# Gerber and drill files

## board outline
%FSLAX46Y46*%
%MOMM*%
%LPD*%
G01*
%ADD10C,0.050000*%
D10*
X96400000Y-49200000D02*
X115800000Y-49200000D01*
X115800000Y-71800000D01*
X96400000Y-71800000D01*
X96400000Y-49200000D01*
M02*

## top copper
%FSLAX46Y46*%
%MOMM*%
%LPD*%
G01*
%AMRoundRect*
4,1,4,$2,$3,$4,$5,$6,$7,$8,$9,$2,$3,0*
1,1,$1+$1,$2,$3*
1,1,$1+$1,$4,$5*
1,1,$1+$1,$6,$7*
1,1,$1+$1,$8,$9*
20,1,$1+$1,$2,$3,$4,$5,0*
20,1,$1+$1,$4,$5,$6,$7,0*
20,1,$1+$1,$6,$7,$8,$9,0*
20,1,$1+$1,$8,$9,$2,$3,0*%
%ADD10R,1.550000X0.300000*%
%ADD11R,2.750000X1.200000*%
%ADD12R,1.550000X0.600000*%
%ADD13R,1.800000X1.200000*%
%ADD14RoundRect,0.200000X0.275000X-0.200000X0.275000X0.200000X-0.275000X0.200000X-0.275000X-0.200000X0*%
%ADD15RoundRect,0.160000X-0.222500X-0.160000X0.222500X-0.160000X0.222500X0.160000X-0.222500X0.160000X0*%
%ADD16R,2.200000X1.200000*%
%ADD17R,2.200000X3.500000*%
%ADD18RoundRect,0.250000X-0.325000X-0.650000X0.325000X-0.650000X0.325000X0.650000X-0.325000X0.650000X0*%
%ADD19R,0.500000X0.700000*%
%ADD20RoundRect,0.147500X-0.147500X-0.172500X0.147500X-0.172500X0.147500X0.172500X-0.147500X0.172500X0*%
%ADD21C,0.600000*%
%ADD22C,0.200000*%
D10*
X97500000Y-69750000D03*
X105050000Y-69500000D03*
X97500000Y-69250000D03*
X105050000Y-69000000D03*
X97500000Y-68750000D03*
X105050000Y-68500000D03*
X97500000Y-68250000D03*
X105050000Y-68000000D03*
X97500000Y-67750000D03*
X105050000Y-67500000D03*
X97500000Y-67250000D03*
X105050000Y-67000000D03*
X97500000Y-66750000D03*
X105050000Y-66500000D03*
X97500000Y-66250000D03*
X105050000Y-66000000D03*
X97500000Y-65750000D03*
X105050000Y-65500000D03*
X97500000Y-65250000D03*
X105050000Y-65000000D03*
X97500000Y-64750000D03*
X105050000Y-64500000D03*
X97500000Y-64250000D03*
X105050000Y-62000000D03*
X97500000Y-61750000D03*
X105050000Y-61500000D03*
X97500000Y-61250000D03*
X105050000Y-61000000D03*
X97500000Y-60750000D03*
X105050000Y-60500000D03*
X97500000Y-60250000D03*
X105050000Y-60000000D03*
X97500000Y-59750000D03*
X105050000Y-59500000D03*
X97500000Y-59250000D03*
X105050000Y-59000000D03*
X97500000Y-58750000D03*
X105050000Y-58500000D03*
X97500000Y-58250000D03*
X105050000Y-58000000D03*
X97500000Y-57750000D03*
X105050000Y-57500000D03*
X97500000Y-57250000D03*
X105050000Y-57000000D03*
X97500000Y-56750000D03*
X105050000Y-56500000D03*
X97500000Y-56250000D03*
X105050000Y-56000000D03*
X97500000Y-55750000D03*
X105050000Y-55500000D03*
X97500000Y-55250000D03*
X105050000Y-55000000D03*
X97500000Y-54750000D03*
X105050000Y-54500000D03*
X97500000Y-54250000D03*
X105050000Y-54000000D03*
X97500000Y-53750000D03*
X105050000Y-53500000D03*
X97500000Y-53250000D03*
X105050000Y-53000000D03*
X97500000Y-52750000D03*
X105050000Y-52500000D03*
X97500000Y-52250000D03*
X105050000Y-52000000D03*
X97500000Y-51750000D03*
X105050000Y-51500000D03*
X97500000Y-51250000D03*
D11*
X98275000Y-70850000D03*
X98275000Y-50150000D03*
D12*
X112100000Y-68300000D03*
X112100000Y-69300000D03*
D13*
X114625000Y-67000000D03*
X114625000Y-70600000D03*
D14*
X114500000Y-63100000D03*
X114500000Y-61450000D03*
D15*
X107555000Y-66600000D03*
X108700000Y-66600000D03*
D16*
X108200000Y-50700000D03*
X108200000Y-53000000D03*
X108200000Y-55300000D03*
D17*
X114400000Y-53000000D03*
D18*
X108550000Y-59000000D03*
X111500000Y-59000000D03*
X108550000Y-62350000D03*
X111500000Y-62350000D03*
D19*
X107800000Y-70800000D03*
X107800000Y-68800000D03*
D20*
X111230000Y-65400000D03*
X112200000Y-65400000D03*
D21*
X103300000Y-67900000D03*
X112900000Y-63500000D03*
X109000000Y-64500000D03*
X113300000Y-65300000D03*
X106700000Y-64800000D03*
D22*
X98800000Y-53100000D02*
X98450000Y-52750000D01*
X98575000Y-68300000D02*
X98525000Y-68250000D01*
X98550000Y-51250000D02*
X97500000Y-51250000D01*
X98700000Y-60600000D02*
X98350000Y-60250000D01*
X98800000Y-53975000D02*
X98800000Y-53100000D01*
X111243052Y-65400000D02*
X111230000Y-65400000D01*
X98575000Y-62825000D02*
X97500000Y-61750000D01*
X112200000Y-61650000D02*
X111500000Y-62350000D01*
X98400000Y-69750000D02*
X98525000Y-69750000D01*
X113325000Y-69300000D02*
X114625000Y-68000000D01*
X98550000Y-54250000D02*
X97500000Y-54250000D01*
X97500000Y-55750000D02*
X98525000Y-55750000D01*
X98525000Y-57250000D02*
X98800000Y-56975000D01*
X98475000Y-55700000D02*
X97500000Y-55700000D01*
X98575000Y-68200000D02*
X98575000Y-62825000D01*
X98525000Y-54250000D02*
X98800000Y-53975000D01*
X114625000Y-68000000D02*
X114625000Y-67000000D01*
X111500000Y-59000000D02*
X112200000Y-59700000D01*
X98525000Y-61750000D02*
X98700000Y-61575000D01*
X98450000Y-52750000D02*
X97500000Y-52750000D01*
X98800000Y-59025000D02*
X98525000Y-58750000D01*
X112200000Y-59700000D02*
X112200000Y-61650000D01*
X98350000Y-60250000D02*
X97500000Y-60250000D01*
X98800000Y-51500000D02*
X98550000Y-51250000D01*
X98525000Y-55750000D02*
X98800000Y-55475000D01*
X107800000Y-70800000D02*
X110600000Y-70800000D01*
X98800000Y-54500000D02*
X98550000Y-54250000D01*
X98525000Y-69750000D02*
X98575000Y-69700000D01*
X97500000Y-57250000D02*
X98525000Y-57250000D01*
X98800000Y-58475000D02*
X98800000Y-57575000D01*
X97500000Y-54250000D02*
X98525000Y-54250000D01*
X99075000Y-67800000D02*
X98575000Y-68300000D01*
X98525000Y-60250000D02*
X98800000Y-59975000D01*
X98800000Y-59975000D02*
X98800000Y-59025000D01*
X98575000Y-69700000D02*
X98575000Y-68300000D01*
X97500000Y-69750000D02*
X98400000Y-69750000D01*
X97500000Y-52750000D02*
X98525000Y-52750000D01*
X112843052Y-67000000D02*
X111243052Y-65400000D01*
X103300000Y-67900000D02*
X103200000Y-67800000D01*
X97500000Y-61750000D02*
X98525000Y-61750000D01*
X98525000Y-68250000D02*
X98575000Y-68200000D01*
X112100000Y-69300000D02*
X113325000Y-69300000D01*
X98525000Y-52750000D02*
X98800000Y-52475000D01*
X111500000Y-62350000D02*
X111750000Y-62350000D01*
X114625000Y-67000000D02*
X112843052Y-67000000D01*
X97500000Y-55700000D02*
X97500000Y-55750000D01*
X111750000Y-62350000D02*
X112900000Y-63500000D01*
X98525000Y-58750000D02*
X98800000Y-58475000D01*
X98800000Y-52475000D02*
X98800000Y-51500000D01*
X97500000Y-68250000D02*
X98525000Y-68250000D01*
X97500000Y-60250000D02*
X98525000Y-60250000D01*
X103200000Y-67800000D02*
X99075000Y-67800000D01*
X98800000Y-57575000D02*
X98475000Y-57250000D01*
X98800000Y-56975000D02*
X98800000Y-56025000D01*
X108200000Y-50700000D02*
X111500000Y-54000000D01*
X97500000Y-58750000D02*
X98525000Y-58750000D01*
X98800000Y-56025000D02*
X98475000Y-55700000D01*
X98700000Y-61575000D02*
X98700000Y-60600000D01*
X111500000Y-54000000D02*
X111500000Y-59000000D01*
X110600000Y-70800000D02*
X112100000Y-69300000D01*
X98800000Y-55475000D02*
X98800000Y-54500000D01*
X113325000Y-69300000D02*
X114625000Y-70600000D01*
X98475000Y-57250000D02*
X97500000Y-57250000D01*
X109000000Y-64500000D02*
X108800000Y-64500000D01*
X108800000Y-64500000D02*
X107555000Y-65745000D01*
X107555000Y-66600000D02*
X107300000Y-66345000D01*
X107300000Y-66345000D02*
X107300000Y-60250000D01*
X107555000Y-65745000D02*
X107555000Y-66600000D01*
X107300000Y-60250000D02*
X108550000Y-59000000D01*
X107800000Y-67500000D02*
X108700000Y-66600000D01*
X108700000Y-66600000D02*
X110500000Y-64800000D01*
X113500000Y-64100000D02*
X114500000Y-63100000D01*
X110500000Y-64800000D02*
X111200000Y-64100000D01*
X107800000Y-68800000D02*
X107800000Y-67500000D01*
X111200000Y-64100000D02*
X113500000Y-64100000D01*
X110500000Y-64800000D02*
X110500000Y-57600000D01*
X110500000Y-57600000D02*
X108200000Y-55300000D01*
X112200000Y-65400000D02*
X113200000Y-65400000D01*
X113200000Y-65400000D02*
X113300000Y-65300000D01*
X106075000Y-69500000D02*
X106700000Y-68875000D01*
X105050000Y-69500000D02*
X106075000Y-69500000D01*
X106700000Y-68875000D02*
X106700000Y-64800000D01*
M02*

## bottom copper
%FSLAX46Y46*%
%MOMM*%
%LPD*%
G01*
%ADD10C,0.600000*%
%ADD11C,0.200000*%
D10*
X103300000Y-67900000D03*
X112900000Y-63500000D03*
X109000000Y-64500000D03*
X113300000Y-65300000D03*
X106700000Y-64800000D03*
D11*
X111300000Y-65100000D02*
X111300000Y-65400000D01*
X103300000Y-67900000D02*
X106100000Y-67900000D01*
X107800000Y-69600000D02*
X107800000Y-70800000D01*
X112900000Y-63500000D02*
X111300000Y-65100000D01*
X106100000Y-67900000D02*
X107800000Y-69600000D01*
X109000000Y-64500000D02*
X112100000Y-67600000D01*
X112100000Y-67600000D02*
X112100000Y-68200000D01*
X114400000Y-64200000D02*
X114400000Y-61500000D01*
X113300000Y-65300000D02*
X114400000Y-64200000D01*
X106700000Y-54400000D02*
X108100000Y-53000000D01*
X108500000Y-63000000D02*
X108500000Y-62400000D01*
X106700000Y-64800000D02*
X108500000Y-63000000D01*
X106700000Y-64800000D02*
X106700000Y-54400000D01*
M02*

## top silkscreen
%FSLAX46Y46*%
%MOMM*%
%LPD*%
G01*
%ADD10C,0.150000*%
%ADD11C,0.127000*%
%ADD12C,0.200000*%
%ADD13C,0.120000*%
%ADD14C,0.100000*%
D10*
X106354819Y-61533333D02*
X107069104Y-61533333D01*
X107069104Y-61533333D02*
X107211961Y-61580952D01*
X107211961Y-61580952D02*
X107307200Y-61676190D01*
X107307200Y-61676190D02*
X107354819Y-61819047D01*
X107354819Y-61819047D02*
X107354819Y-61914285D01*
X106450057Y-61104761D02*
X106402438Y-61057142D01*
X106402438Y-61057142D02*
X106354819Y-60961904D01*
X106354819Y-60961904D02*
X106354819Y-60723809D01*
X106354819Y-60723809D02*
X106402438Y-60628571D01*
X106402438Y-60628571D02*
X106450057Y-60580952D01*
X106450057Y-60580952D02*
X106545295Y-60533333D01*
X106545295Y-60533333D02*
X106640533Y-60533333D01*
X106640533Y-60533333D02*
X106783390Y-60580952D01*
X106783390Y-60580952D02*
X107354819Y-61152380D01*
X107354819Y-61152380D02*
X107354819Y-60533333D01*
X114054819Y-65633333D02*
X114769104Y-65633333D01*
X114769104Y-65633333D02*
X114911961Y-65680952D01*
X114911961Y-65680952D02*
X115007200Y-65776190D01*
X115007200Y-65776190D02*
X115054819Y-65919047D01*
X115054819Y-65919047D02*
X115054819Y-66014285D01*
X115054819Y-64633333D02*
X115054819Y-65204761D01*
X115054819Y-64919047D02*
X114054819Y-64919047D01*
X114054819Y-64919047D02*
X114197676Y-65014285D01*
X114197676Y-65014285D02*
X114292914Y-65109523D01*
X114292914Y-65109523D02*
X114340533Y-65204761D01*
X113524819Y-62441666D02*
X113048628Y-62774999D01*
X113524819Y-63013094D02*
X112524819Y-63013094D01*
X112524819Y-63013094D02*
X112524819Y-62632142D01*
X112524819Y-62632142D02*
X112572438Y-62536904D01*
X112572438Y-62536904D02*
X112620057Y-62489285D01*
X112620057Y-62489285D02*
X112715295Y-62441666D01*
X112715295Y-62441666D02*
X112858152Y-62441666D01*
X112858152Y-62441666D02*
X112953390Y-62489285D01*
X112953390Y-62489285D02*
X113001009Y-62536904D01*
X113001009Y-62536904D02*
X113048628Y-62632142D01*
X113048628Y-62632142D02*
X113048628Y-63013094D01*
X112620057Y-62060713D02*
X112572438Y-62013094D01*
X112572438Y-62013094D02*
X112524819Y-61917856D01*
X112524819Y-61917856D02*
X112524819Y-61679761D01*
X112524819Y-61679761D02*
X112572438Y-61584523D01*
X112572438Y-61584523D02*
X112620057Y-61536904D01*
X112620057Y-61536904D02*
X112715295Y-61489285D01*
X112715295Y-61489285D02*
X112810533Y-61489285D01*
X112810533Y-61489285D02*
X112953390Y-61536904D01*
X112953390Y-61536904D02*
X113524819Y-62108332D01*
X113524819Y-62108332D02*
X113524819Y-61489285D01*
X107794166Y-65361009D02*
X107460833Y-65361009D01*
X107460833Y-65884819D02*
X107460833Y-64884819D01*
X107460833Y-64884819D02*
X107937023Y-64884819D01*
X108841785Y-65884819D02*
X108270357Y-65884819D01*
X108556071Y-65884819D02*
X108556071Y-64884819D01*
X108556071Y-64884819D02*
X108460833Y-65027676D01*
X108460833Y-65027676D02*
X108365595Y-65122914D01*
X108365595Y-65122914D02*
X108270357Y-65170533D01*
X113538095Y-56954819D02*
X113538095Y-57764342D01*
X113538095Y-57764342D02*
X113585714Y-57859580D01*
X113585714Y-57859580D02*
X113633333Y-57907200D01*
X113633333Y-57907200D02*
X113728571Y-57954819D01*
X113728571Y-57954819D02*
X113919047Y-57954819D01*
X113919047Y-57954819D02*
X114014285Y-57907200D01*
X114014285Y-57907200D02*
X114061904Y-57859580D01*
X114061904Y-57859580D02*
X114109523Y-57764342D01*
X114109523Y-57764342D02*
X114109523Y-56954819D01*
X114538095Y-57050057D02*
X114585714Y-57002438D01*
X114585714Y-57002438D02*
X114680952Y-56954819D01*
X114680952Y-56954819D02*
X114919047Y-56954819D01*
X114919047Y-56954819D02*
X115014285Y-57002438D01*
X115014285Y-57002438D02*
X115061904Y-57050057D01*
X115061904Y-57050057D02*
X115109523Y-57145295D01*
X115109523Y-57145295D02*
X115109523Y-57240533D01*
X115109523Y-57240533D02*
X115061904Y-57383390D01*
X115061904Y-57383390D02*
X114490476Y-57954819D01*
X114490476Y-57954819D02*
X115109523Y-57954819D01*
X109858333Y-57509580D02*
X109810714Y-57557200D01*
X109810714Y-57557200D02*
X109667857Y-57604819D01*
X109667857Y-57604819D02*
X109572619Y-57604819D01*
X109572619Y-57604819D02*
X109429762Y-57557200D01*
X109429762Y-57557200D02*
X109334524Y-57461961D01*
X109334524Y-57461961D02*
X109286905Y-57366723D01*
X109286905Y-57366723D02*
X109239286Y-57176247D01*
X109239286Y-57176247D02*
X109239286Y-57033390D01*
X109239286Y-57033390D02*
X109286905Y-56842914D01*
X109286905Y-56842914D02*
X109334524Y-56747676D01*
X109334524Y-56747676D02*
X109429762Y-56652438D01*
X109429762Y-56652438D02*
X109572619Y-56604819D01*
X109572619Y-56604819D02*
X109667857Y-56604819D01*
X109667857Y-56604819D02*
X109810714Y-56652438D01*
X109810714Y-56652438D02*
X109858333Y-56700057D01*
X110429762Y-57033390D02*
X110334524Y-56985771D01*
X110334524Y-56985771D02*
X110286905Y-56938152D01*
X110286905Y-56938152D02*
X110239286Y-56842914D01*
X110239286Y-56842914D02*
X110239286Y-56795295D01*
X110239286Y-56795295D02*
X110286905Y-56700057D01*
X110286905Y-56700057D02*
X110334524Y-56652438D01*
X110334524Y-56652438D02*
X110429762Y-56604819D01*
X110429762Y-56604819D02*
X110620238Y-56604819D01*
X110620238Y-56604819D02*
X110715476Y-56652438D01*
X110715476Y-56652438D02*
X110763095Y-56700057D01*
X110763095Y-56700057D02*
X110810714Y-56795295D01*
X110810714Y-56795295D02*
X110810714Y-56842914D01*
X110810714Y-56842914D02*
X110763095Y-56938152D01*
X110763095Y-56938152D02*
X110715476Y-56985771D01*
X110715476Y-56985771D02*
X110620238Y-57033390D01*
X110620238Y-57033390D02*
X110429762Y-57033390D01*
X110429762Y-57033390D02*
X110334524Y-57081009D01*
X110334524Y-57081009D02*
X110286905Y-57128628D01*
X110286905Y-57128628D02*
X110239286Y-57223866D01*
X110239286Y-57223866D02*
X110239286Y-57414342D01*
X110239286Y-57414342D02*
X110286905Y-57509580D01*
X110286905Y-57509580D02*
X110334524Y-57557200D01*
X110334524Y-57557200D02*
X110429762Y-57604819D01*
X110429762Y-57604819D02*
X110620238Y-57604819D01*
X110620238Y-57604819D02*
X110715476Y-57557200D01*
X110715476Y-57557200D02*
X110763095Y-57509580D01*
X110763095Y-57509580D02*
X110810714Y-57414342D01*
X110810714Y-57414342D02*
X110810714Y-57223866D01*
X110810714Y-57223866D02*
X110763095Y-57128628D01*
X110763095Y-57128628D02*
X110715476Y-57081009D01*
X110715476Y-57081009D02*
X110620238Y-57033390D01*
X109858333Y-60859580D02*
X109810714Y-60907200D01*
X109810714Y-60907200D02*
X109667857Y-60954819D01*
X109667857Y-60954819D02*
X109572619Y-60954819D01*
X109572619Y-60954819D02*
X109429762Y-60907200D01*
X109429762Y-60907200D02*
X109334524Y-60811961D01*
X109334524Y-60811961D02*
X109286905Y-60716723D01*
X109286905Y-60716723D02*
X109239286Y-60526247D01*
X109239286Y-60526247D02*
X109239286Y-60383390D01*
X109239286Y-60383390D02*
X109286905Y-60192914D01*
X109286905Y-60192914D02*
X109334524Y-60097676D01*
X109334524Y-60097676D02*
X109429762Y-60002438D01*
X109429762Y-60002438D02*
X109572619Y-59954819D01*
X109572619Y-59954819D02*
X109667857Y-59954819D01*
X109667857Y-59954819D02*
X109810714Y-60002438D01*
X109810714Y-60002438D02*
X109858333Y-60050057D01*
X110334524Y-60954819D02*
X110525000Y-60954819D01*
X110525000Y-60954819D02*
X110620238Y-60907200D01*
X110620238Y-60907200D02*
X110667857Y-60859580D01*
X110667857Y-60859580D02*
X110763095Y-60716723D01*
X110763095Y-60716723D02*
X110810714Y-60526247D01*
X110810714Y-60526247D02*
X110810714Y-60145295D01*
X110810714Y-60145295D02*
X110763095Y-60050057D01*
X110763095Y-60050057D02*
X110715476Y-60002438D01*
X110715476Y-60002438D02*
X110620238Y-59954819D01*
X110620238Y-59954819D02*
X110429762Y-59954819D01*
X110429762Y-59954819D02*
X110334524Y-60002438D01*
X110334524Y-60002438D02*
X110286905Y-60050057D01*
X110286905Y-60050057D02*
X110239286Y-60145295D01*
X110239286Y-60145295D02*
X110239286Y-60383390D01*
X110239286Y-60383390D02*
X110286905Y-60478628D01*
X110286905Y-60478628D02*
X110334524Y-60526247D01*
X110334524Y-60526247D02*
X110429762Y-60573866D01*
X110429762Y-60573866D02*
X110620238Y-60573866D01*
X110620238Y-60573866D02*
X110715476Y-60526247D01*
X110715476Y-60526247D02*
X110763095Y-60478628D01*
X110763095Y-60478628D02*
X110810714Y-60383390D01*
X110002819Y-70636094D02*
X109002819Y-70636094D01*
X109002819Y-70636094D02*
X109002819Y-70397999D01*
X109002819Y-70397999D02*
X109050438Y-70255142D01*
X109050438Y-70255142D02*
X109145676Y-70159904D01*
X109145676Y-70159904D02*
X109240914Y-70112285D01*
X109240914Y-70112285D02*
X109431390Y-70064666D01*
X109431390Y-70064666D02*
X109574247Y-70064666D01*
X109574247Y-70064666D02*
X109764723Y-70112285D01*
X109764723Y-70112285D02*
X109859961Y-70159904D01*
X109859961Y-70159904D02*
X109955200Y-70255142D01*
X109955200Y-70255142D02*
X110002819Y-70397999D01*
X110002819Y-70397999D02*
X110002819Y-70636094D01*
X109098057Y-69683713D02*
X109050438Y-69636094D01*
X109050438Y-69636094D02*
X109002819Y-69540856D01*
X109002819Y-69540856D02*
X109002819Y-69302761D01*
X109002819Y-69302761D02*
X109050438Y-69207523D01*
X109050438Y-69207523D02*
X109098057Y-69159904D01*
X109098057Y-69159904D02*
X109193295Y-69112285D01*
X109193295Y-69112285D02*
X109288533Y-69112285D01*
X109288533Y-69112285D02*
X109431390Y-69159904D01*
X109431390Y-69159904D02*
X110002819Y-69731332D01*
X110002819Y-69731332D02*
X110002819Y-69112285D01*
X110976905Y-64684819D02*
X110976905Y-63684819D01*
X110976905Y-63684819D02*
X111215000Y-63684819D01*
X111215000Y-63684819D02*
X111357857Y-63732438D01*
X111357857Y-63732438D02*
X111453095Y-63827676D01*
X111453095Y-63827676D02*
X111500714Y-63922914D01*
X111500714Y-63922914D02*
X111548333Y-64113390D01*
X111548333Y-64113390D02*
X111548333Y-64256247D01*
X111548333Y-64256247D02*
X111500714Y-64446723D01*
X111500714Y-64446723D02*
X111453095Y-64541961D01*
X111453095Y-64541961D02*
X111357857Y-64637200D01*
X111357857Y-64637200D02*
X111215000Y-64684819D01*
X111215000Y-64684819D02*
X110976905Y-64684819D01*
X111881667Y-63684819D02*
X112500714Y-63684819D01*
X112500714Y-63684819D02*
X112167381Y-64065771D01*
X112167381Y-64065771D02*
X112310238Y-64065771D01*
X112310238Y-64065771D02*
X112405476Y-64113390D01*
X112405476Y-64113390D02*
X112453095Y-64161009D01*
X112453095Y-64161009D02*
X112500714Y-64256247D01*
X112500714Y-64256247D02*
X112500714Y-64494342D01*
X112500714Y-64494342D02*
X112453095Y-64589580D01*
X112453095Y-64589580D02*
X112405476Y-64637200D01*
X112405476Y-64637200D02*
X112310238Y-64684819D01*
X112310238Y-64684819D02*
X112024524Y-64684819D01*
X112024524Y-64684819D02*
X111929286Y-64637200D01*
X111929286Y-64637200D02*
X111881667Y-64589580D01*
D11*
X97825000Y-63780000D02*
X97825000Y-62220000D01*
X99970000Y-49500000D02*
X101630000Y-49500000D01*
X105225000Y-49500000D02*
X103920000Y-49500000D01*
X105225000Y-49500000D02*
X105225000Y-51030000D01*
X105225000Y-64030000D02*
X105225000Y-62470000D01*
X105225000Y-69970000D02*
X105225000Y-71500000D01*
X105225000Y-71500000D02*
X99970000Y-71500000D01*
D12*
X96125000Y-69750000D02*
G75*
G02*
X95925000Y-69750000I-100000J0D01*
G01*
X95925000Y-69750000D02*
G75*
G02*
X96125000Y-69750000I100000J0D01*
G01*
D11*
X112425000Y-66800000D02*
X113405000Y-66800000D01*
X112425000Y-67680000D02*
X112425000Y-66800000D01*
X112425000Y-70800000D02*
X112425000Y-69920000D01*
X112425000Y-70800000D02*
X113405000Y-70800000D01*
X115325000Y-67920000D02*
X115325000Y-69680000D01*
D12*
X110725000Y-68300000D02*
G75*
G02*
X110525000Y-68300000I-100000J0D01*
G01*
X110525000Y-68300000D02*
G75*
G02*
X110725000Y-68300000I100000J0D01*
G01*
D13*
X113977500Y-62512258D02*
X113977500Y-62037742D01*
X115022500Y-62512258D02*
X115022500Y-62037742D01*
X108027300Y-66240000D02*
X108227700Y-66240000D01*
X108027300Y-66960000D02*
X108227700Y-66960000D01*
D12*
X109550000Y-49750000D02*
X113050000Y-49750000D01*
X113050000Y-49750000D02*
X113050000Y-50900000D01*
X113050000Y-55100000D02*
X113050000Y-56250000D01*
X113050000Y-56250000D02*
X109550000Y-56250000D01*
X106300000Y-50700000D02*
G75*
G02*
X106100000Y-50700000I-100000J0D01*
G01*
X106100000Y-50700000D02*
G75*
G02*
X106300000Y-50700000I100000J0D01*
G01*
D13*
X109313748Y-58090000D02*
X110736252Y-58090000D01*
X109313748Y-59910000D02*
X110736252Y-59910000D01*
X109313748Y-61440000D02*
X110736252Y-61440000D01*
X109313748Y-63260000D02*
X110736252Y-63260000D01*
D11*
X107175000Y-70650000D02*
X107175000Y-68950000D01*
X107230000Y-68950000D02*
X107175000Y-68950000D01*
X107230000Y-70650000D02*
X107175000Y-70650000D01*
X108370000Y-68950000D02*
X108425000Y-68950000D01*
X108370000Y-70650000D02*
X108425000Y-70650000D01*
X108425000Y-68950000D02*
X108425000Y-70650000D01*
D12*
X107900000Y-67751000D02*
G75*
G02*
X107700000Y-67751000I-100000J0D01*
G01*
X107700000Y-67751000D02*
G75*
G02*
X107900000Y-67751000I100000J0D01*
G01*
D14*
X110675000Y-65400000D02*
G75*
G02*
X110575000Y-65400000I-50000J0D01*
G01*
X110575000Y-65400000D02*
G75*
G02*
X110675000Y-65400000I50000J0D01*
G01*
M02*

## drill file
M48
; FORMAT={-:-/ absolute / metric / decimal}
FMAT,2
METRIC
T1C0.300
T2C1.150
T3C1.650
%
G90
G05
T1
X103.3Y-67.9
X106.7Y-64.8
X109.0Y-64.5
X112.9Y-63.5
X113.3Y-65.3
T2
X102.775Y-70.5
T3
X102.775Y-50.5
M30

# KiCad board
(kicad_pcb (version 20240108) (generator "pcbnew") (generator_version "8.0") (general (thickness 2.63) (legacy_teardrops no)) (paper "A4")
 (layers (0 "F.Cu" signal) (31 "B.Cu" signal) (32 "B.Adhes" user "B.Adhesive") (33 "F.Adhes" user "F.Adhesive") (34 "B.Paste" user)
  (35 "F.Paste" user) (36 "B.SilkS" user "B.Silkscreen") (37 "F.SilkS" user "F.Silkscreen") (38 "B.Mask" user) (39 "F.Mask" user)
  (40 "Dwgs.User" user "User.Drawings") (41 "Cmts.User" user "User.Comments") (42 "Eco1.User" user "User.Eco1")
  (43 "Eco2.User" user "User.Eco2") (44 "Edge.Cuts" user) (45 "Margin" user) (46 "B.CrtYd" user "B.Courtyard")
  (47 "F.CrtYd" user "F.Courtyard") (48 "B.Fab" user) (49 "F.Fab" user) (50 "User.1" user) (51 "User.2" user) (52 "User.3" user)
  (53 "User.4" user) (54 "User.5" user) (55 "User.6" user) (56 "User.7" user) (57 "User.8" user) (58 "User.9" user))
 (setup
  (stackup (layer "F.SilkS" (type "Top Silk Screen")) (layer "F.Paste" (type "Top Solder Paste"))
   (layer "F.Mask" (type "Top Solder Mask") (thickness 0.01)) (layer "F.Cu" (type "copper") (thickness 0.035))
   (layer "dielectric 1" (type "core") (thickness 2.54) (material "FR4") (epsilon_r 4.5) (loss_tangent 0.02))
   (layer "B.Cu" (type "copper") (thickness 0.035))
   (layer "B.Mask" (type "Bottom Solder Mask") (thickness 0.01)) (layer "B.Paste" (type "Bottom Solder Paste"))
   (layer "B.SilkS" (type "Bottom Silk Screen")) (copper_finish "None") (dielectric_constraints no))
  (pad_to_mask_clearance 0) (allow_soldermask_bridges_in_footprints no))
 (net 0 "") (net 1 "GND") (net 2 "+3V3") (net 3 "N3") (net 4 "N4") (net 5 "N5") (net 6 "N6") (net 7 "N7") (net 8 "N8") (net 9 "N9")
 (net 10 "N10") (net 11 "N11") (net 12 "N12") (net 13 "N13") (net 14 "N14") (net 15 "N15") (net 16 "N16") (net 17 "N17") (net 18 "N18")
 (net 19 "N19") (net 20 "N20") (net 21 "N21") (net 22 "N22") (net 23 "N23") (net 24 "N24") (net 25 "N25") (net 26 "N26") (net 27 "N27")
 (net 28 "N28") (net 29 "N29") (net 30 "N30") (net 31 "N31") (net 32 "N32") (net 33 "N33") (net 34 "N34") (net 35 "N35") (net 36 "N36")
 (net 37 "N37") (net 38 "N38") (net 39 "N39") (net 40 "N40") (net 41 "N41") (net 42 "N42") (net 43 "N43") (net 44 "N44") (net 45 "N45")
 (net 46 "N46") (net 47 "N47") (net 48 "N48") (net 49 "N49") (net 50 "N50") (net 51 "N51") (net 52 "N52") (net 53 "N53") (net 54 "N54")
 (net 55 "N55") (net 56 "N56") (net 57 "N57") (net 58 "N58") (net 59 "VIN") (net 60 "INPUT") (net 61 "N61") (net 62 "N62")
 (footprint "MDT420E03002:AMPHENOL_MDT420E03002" (layer "F.Cu") (at 102.775 60.5 90)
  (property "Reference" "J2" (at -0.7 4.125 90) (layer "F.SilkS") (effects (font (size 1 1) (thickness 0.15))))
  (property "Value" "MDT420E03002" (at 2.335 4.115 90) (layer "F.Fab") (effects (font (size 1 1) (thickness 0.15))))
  (fp_line (start -3.28 -4.95) (end -1.72 -4.95) (stroke (width 0.127) (type solid)) (layer "F.SilkS"))
  (fp_line (start 11 -2.805) (end 11 -1.145) (stroke (width 0.127) (type solid)) (layer "F.SilkS"))
  (fp_line (start 11 2.45) (end 11 1.145) (stroke (width 0.127) (type solid)) (layer "F.SilkS"))
  (fp_line (start 11 2.45) (end 9.47 2.45) (stroke (width 0.127) (type solid)) (layer "F.SilkS"))
  (fp_line (start -3.53 2.45) (end -1.97 2.45) (stroke (width 0.127) (type solid)) (layer "F.SilkS"))
  (fp_line (start -9.47 2.45) (end -11 2.45) (stroke (width 0.127) (type solid)) (layer "F.SilkS"))
  (fp_line (start -11 2.45) (end -11 -2.805) (stroke (width 0.127) (type solid)) (layer "F.SilkS"))
  (fp_circle (center -9.25 -6.75) (end -9.15 -6.75) (stroke (width 0.2) (type solid)) (fill none) (layer "F.SilkS"))
  (pad "" np_thru_hole circle (at -10 0 90) (size 1.15 1.15) (drill 1.15) (layers "*.Cu" "*.Mask"))
  (pad "" np_thru_hole circle (at 10 0 90) (size 1.65 1.65) (drill 1.65) (layers "*.Cu" "*.Mask"))
  (pad "1" smd rect (at -9.25 -5.275 90) (size 0.3 1.55) (layers "F.Cu" "F.Paste" "F.Mask") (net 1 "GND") (solder_mask_margin 0.102))
  (pad "2" smd rect (at -9 2.275 90) (size 0.3 1.55) (layers "F.Cu" "F.Paste" "F.Mask") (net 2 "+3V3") (solder_mask_margin 0.102))
  (pad "3" smd rect (at -8.75 -5.275 90) (size 0.3 1.55) (layers "F.Cu" "F.Paste" "F.Mask") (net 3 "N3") (solder_mask_margin 0.102))
  (pad "4" smd rect (at -8.5 2.275 90) (size 0.3 1.55) (layers "F.Cu" "F.Paste" "F.Mask") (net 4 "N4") (solder_mask_margin 0.102))
  (pad "5" smd rect (at -8.25 -5.275 90) (size 0.3 1.55) (layers "F.Cu" "F.Paste" "F.Mask") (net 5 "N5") (solder_mask_margin 0.102))
  (pad "6" smd rect (at -8 2.275 90) (size 0.3 1.55) (layers "F.Cu" "F.Paste" "F.Mask") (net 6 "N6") (solder_mask_margin 0.102))
  (pad "7" smd rect (at -7.75 -5.275 90) (size 0.3 1.55) (layers "F.Cu" "F.Paste" "F.Mask") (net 1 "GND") (solder_mask_margin 0.102))
  (pad "8" smd rect (at -7.5 2.275 90) (size 0.3 1.55) (layers "F.Cu" "F.Paste" "F.Mask") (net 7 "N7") (solder_mask_margin 0.102))
  (pad "9" smd rect (at -7.25 -5.275 90) (size 0.3 1.55) (layers "F.Cu" "F.Paste" "F.Mask") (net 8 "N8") (solder_mask_margin 0.102))
  (pad "10" smd rect (at -7 2.275 90) (size 0.3 1.55) (layers "F.Cu" "F.Paste" "F.Mask") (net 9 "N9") (solder_mask_margin 0.102))
  (pad "11" smd rect (at -6.75 -5.275 90) (size 0.3 1.55) (layers "F.Cu" "F.Paste" "F.Mask") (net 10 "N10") (solder_mask_margin 0.102))
  (pad "12" smd rect (at -6.5 2.275 90) (size 0.3 1.55) (layers "F.Cu" "F.Paste" "F.Mask") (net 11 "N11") (solder_mask_margin 0.102))
  (pad "13" smd rect (at -6.25 -5.275 90) (size 0.3 1.55) (layers "F.Cu" "F.Paste" "F.Mask") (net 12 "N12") (solder_mask_margin 0.102))
  (pad "14" smd rect (at -6 2.275 90) (size 0.3 1.55) (layers "F.Cu" "F.Paste" "F.Mask") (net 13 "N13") (solder_mask_margin 0.102))
  (pad "15" smd rect (at -5.75 -5.275 90) (size 0.3 1.55) (layers "F.Cu" "F.Paste" "F.Mask") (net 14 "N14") (solder_mask_margin 0.102))
  (pad "16" smd rect (at -5.5 2.275 90) (size 0.3 1.55) (layers "F.Cu" "F.Paste" "F.Mask") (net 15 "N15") (solder_mask_margin 0.102))
  (pad "17" smd rect (at -5.25 -5.275 90) (size 0.3 1.55) (layers "F.Cu" "F.Paste" "F.Mask") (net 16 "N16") (solder_mask_margin 0.102))
  (pad "18" smd rect (at -5 2.275 90) (size 0.3 1.55) (layers "F.Cu" "F.Paste" "F.Mask") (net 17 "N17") (solder_mask_margin 0.102))
  (pad "19" smd rect (at -4.75 -5.275 90) (size 0.3 1.55) (layers "F.Cu" "F.Paste" "F.Mask") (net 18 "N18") (solder_mask_margin 0.102))
  (pad "20" smd rect (at -4.5 2.275 90) (size 0.3 1.55) (layers "F.Cu" "F.Paste" "F.Mask") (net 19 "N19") (solder_mask_margin 0.102))
  (pad "21" smd rect (at -4.25 -5.275 90) (size 0.3 1.55) (layers "F.Cu" "F.Paste" "F.Mask") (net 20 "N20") (solder_mask_margin 0.102))
  (pad "22" smd rect (at -4 2.275 90) (size 0.3 1.55) (layers "F.Cu" "F.Paste" "F.Mask") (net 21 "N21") (solder_mask_margin 0.102))
  (pad "23" smd rect (at -3.75 -5.275 90) (size 0.3 1.55) (layers "F.Cu" "F.Paste" "F.Mask") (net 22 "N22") (solder_mask_margin 0.102))
  (pad "32" smd rect (at -1.5 2.275 90) (size 0.3 1.55) (layers "F.Cu" "F.Paste" "F.Mask") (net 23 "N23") (solder_mask_margin 0.102))
  (pad "33" smd rect (at -1.25 -5.275 90) (size 0.3 1.55) (layers "F.Cu" "F.Paste" "F.Mask") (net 1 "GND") (solder_mask_margin 0.102))
  (pad "34" smd rect (at -1 2.275 90) (size 0.3 1.55) (layers "F.Cu" "F.Paste" "F.Mask") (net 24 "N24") (solder_mask_margin 0.102))
  (pad "35" smd rect (at -0.75 -5.275 90) (size 0.3 1.55) (layers "F.Cu" "F.Paste" "F.Mask") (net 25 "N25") (solder_mask_margin 0.102))
  (pad "36" smd rect (at -0.5 2.275 90) (size 0.3 1.55) (layers "F.Cu" "F.Paste" "F.Mask") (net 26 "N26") (solder_mask_margin 0.102))
  (pad "37" smd rect (at -0.25 -5.275 90) (size 0.3 1.55) (layers "F.Cu" "F.Paste" "F.Mask") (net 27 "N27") (solder_mask_margin 0.102))
  (pad "38" smd rect (at 0 2.275 90) (size 0.3 1.55) (layers "F.Cu" "F.Paste" "F.Mask") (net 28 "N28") (solder_mask_margin 0.102))
  (pad "39" smd rect (at 0.25 -5.275 90) (size 0.3 1.55) (layers "F.Cu" "F.Paste" "F.Mask") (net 1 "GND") (solder_mask_margin 0.102))
  (pad "40" smd rect (at 0.5 2.275 90) (size 0.3 1.55) (layers "F.Cu" "F.Paste" "F.Mask") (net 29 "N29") (solder_mask_margin 0.102))
  (pad "41" smd rect (at 0.75 -5.275 90) (size 0.3 1.55) (layers "F.Cu" "F.Paste" "F.Mask") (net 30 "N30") (solder_mask_margin 0.102))
  (pad "42" smd rect (at 1 2.275 90) (size 0.3 1.55) (layers "F.Cu" "F.Paste" "F.Mask") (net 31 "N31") (solder_mask_margin 0.102))
  (pad "43" smd rect (at 1.25 -5.275 90) (size 0.3 1.55) (layers "F.Cu" "F.Paste" "F.Mask") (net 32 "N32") (solder_mask_margin 0.102))
  (pad "44" smd rect (at 1.5 2.275 90) (size 0.3 1.55) (layers "F.Cu" "F.Paste" "F.Mask") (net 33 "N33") (solder_mask_margin 0.102))
  (pad "45" smd rect (at 1.75 -5.275 90) (size 0.3 1.55) (layers "F.Cu" "F.Paste" "F.Mask") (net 1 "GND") (solder_mask_margin 0.102))
  (pad "46" smd rect (at 2 2.275 90) (size 0.3 1.55) (layers "F.Cu" "F.Paste" "F.Mask") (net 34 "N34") (solder_mask_margin 0.102))
  (pad "47" smd rect (at 2.25 -5.275 90) (size 0.3 1.55) (layers "F.Cu" "F.Paste" "F.Mask") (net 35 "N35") (solder_mask_margin 0.102))
  (pad "48" smd rect (at 2.5 2.275 90) (size 0.3 1.55) (layers "F.Cu" "F.Paste" "F.Mask") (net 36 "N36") (solder_mask_margin 0.102))
  (pad "49" smd rect (at 2.75 -5.275 90) (size 0.3 1.55) (layers "F.Cu" "F.Paste" "F.Mask") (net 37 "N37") (solder_mask_margin 0.102))
  (pad "50" smd rect (at 3 2.275 90) (size 0.3 1.55) (layers "F.Cu" "F.Paste" "F.Mask") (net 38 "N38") (solder_mask_margin 0.102))
  (pad "51" smd rect (at 3.25 -5.275 90) (size 0.3 1.55) (layers "F.Cu" "F.Paste" "F.Mask") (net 1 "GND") (solder_mask_margin 0.102))
  (pad "52" smd rect (at 3.5 2.275 90) (size 0.3 1.55) (layers "F.Cu" "F.Paste" "F.Mask") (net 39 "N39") (solder_mask_margin 0.102))
  (pad "53" smd rect (at 3.75 -5.275 90) (size 0.3 1.55) (layers "F.Cu" "F.Paste" "F.Mask") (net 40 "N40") (solder_mask_margin 0.102))
  (pad "54" smd rect (at 4 2.275 90) (size 0.3 1.55) (layers "F.Cu" "F.Paste" "F.Mask") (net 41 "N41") (solder_mask_margin 0.102))
  (pad "55" smd rect (at 4.25 -5.275 90) (size 0.3 1.55) (layers "F.Cu" "F.Paste" "F.Mask") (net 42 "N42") (solder_mask_margin 0.102))
  (pad "56" smd rect (at 4.5 2.275 90) (size 0.3 1.55) (layers "F.Cu" "F.Paste" "F.Mask") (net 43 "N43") (solder_mask_margin 0.102))
  (pad "57" smd rect (at 4.75 -5.275 90) (size 0.3 1.55) (layers "F.Cu" "F.Paste" "F.Mask") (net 1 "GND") (solder_mask_margin 0.102))
  (pad "58" smd rect (at 5 2.275 90) (size 0.3 1.55) (layers "F.Cu" "F.Paste" "F.Mask") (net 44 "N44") (solder_mask_margin 0.102))
  (pad "59" smd rect (at 5.25 -5.275 90) (size 0.3 1.55) (layers "F.Cu" "F.Paste" "F.Mask") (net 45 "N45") (solder_mask_margin 0.102))
  (pad "60" smd rect (at 5.5 2.275 90) (size 0.3 1.55) (layers "F.Cu" "F.Paste" "F.Mask") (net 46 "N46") (solder_mask_margin 0.102))
  (pad "61" smd rect (at 5.75 -5.275 90) (size 0.3 1.55) (layers "F.Cu" "F.Paste" "F.Mask") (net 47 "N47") (solder_mask_margin 0.102))
  (pad "62" smd rect (at 6 2.275 90) (size 0.3 1.55) (layers "F.Cu" "F.Paste" "F.Mask") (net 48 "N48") (solder_mask_margin 0.102))
  (pad "63" smd rect (at 6.25 -5.275 90) (size 0.3 1.55) (layers "F.Cu" "F.Paste" "F.Mask") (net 1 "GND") (solder_mask_margin 0.102))
  (pad "64" smd rect (at 6.5 2.275 90) (size 0.3 1.55) (layers "F.Cu" "F.Paste" "F.Mask") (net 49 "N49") (solder_mask_margin 0.102))
  (pad "65" smd rect (at 6.75 -5.275 90) (size 0.3 1.55) (layers "F.Cu" "F.Paste" "F.Mask") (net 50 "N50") (solder_mask_margin 0.102))
  (pad "66" smd rect (at 7 2.275 90) (size 0.3 1.55) (layers "F.Cu" "F.Paste" "F.Mask") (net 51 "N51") (solder_mask_margin 0.102))
  (pad "67" smd rect (at 7.25 -5.275 90) (size 0.3 1.55) (layers "F.Cu" "F.Paste" "F.Mask") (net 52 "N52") (solder_mask_margin 0.102))
  (pad "68" smd rect (at 7.5 2.275 90) (size 0.3 1.55) (layers "F.Cu" "F.Paste" "F.Mask") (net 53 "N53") (solder_mask_margin 0.102))
  (pad "69" smd rect (at 7.75 -5.275 90) (size 0.3 1.55) (layers "F.Cu" "F.Paste" "F.Mask") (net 1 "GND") (solder_mask_margin 0.102))
  (pad "70" smd rect (at 8 2.275 90) (size 0.3 1.55) (layers "F.Cu" "F.Paste" "F.Mask") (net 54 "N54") (solder_mask_margin 0.102))
  (pad "71" smd rect (at 8.25 -5.275 90) (size 0.3 1.55) (layers "F.Cu" "F.Paste" "F.Mask") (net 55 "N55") (solder_mask_margin 0.102))
  (pad "72" smd rect (at 8.5 2.275 90) (size 0.3 1.55) (layers "F.Cu" "F.Paste" "F.Mask") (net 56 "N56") (solder_mask_margin 0.102))
  (pad "73" smd rect (at 8.75 -5.275 90) (size 0.3 1.55) (layers "F.Cu" "F.Paste" "F.Mask") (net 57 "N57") (solder_mask_margin 0.102))
  (pad "74" smd rect (at 9 2.275 90) (size 0.3 1.55) (layers "F.Cu" "F.Paste" "F.Mask") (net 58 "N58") (solder_mask_margin 0.102))
  (pad "75" smd rect (at 9.25 -5.275 90) (size 0.3 1.55) (layers "F.Cu" "F.Paste" "F.Mask") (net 1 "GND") (solder_mask_margin 0.102))
  (pad "SH1" smd rect (at -10.35 -4.5 90) (size 1.2 2.75) (layers "F.Cu" "F.Paste" "F.Mask") (solder_mask_margin 0.102))
  (pad "SH2" smd rect (at 10.35 -4.5 90) (size 1.2 2.75) (layers "F.Cu" "F.Paste" "F.Mask") (solder_mask_margin 0.102)))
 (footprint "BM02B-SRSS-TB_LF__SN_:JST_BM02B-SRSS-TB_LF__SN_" (layer "F.Cu") (at 114.625 68.8 -90)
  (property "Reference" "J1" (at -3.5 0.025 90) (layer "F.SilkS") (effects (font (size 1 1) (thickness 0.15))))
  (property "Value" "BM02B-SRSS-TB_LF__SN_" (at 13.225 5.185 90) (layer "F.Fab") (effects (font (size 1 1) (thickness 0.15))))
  (fp_line (start -2 2.2) (end -2 1.22) (stroke (width 0.127) (type solid)) (layer "F.SilkS"))
  (fp_line (start -1.12 2.2) (end -2 2.2) (stroke (width 0.127) (type solid)) (layer "F.SilkS"))
  (fp_line (start 2 2.2) (end 1.12 2.2) (stroke (width 0.127) (type solid)) (layer "F.SilkS"))
  (fp_line (start 2 2.2) (end 2 1.22) (stroke (width 0.127) (type solid)) (layer "F.SilkS"))
  (fp_line (start -0.88 -0.7) (end 0.88 -0.7) (stroke (width 0.127) (type solid)) (layer "F.SilkS"))
  (fp_circle (center -0.5 4) (end -0.4 4) (stroke (width 0.2) (type solid)) (fill none) (layer "F.SilkS"))
  (pad "1" smd rect (at -0.5 2.525 270) (size 0.6 1.55) (layers "F.Cu" "F.Paste" "F.Mask") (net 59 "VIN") (solder_mask_margin 0.102))
  (pad "2" smd rect (at 0.5 2.525 270) (size 0.6 1.55) (layers "F.Cu" "F.Paste" "F.Mask") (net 1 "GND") (solder_mask_margin 0.102))
  (pad "S1" smd rect (at -1.8 0 270) (size 1.2 1.8) (layers "F.Cu" "F.Paste" "F.Mask") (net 1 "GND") (solder_mask_margin 0.102))
  (pad "S2" smd rect (at 1.8 0 270) (size 1.2 1.8) (layers "F.Cu" "F.Paste" "F.Mask") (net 1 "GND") (solder_mask_margin 0.102)))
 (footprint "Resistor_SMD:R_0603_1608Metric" (layer "F.Cu") (at 114.5 62.275 90)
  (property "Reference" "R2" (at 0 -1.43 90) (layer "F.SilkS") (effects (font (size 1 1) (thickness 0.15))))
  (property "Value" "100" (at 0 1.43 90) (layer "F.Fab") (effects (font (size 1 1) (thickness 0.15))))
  (fp_line (start -0.237258 -0.5225) (end 0.237258 -0.5225) (stroke (width 0.12) (type solid)) (layer "F.SilkS"))
  (fp_line (start -0.237258 0.5225) (end 0.237258 0.5225) (stroke (width 0.12) (type solid)) (layer "F.SilkS"))
  (pad "1" smd roundrect (at -0.825 0 90) (size 0.8 0.95) (layers "F.Cu" "F.Paste" "F.Mask") (roundrect_rratio 0.25) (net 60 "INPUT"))
  (pad "2" smd roundrect (at 0.825 0 90) (size 0.8 0.95) (layers "F.Cu" "F.Paste" "F.Mask") (roundrect_rratio 0.25) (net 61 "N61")))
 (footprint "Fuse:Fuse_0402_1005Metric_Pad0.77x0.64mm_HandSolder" (layer "F.Cu") (at 108.1275 66.6)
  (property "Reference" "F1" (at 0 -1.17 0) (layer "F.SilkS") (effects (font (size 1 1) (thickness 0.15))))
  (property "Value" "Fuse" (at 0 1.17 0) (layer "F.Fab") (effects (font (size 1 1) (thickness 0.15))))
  (fp_line (start -0.1002 -0.36) (end 0.1002 -0.36) (stroke (width 0.12) (type solid)) (layer "F.SilkS"))
  (fp_line (start -0.1002 0.36) (end 0.1002 0.36) (stroke (width 0.12) (type solid)) (layer "F.SilkS"))
  (pad "1" smd roundrect (at -0.5725 0) (size 0.765 0.64) (layers "F.Cu" "F.Paste" "F.Mask") (roundrect_rratio 0.25) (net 59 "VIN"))
  (pad "2" smd roundrect (at 0.5725 0) (size 0.765 0.64) (layers "F.Cu" "F.Paste" "F.Mask") (roundrect_rratio 0.25) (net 60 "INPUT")))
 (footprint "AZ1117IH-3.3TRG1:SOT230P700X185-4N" (layer "F.Cu") (at 111.3 53)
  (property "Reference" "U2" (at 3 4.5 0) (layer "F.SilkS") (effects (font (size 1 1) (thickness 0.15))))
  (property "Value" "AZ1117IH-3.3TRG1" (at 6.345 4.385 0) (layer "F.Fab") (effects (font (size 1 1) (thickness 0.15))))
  (fp_line (start -1.75 -3.25) (end 1.75 -3.25) (stroke (width 0.2) (type solid)) (layer "F.SilkS"))
  (fp_line (start 1.75 -3.25) (end 1.75 -2.1) (stroke (width 0.2) (type solid)) (layer "F.SilkS"))
  (fp_line (start 1.75 2.1) (end 1.75 3.25) (stroke (width 0.2) (type solid)) (layer "F.SilkS"))
  (fp_line (start 1.75 3.25) (end -1.75 3.25) (stroke (width 0.2) (type solid)) (layer "F.SilkS"))
  (fp_circle (center -5.1 -2.3) (end -5 -2.3) (stroke (width 0.2) (type solid)) (fill none) (layer "F.SilkS"))
  (pad "1" smd rect (at -3.1 -2.3) (size 2.2 1.2) (layers "F.Cu" "F.Paste" "F.Mask") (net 1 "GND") (solder_mask_margin 0.102))
  (pad "2" smd rect (at -3.1 0) (size 2.2 1.2) (layers "F.Cu" "F.Paste" "F.Mask") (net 2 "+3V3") (solder_mask_margin 0.102))
  (pad "3" smd rect (at -3.1 2.3) (size 2.2 1.2) (layers "F.Cu" "F.Paste" "F.Mask") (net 60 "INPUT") (solder_mask_margin 0.102))
  (pad "4" smd rect (at 3.1 0) (size 2.2 3.5) (layers "F.Cu" "F.Paste" "F.Mask") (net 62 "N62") (solder_mask_margin 0.102)))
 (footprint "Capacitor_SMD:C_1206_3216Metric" (layer "F.Cu") (at 110.025 59)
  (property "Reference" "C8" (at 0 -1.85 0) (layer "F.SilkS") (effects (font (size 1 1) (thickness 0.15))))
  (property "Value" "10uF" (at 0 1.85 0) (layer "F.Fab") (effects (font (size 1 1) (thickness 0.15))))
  (fp_line (start -0.711252 -0.91) (end 0.711252 -0.91) (stroke (width 0.12) (type solid)) (layer "F.SilkS"))
  (fp_line (start -0.711252 0.91) (end 0.711252 0.91) (stroke (width 0.12) (type solid)) (layer "F.SilkS"))
  (pad "1" smd roundrect (at -1.475 0) (size 1.15 1.8) (layers "F.Cu" "F.Paste" "F.Mask") (roundrect_rratio 0.217391) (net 59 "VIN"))
  (pad "2" smd roundrect (at 1.475 0) (size 1.15 1.8) (layers "F.Cu" "F.Paste" "F.Mask") (roundrect_rratio 0.217391) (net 1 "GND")))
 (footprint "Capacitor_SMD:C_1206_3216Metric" (layer "F.Cu") (at 110.025 62.35)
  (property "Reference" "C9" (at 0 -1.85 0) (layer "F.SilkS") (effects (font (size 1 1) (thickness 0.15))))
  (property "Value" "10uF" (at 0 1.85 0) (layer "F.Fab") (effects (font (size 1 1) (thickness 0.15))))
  (fp_line (start -0.711252 -0.91) (end 0.711252 -0.91) (stroke (width 0.12) (type solid)) (layer "F.SilkS"))
  (fp_line (start -0.711252 0.91) (end 0.711252 0.91) (stroke (width 0.12) (type solid)) (layer "F.SilkS"))
  (pad "1" smd roundrect (at -1.475 0) (size 1.15 1.8) (layers "F.Cu" "F.Paste" "F.Mask") (roundrect_rratio 0.217391) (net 2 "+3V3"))
  (pad "2" smd roundrect (at 1.475 0) (size 1.15 1.8) (layers "F.Cu" "F.Paste" "F.Mask") (roundrect_rratio 0.217391) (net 1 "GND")))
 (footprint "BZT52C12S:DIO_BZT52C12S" (layer "F.Cu") (at 107.8 69.8 -90)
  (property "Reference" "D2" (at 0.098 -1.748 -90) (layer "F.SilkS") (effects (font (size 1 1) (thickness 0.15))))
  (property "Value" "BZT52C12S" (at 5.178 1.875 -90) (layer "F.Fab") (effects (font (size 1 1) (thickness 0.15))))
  (fp_line (start 0.85 0.625) (end -0.85 0.625) (stroke (width 0.127) (type solid)) (layer "F.SilkS"))
  (fp_line (start -0.85 0.57) (end -0.85 0.625) (stroke (width 0.127) (type solid)) (layer "F.SilkS"))
  (fp_line (start 0.85 0.57) (end 0.85 0.625) (stroke (width 0.127) (type solid)) (layer "F.SilkS"))
  (fp_line (start -0.85 -0.57) (end -0.85 -0.625) (stroke (width 0.127) (type solid)) (layer "F.SilkS"))
  (fp_line (start 0.85 -0.57) (end 0.85 -0.625) (stroke (width 0.127) (type solid)) (layer "F.SilkS"))
  (fp_line (start -0.85 -0.625) (end 0.85 -0.625) (stroke (width 0.127) (type solid)) (layer "F.SilkS"))
  (fp_circle (center -2.049 0) (end -1.949 0) (stroke (width 0.2) (type solid)) (fill none) (layer "F.SilkS"))
  (pad "A" smd rect (at 1 0 270) (size 0.7 0.5) (layers "F.Cu" "F.Paste" "F.Mask") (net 1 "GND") (solder_mask_margin 0.102))
  (pad "C" smd rect (at -1 0 270) (size 0.7 0.5) (layers "F.Cu" "F.Paste" "F.Mask") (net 60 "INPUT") (solder_mask_margin 0.102)))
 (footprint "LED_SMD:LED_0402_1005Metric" (layer "F.Cu") (at 111.715 65.4)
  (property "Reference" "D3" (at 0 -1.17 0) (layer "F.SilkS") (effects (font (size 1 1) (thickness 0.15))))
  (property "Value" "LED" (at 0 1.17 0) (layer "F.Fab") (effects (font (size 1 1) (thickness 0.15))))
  (fp_circle (center -1.09 0) (end -1.04 0) (stroke (width 0.1) (type solid)) (fill none) (layer "F.SilkS"))
  (pad "1" smd roundrect (at -0.485 0) (size 0.59 0.64) (layers "F.Cu" "F.Paste" "F.Mask") (roundrect_rratio 0.25) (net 1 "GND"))
  (pad "2" smd roundrect (at 0.485 0) (size 0.59 0.64) (layers "F.Cu" "F.Paste" "F.Mask") (roundrect_rratio 0.25) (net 61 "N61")))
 (gr_rect (start 96.4 49.2) (end 115.8 71.8) (stroke (width 0.05) (type default)) (fill none) (layer "Edge.Cuts"))
 (segment (start 98.8 53.1) (end 98.45 52.75) (width 0.2) (layer "F.Cu") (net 1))
 (segment (start 98.575 68.3) (end 98.525 68.25) (width 0.2) (layer "F.Cu") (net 1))
 (segment (start 98.55 51.25) (end 97.5 51.25) (width 0.2) (layer "F.Cu") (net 1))
 (segment (start 98.7 60.6) (end 98.35 60.25) (width 0.2) (layer "F.Cu") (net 1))
 (segment (start 98.8 53.975) (end 98.8 53.1) (width 0.2) (layer "F.Cu") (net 1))
 (segment (start 111.243052 65.4) (end 111.23 65.4) (width 0.2) (layer "F.Cu") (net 1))
 (segment (start 98.575 62.825) (end 97.5 61.75) (width 0.2) (layer "F.Cu") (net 1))
 (segment (start 112.2 61.65) (end 111.5 62.35) (width 0.2) (layer "F.Cu") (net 1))
 (segment (start 98.4 69.75) (end 98.525 69.75) (width 0.2) (layer "F.Cu") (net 1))
 (segment (start 113.325 69.3) (end 114.625 68) (width 0.2) (layer "F.Cu") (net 1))
 (segment (start 98.55 54.25) (end 97.5 54.25) (width 0.2) (layer "F.Cu") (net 1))
 (segment (start 97.5 55.75) (end 98.525 55.75) (width 0.2) (layer "F.Cu") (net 1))
 (segment (start 98.525 57.25) (end 98.8 56.975) (width 0.2) (layer "F.Cu") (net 1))
 (segment (start 98.475 55.7) (end 97.5 55.7) (width 0.2) (layer "F.Cu") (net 1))
 (segment (start 98.575 68.2) (end 98.575 62.825) (width 0.2) (layer "F.Cu") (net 1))
 (segment (start 98.525 54.25) (end 98.8 53.975) (width 0.2) (layer "F.Cu") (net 1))
 (segment (start 114.625 68) (end 114.625 67) (width 0.2) (layer "F.Cu") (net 1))
 (segment (start 111.5 59) (end 112.2 59.7) (width 0.2) (layer "F.Cu") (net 1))
 (segment (start 98.525 61.75) (end 98.7 61.575) (width 0.2) (layer "F.Cu") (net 1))
 (segment (start 98.45 52.75) (end 97.5 52.75) (width 0.2) (layer "F.Cu") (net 1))
 (segment (start 98.8 59.025) (end 98.525 58.75) (width 0.2) (layer "F.Cu") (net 1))
 (segment (start 112.2 59.7) (end 112.2 61.65) (width 0.2) (layer "F.Cu") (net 1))
 (segment (start 98.35 60.25) (end 97.5 60.25) (width 0.2) (layer "F.Cu") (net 1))
 (segment (start 98.8 51.5) (end 98.55 51.25) (width 0.2) (layer "F.Cu") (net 1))
 (segment (start 98.525 55.75) (end 98.8 55.475) (width 0.2) (layer "F.Cu") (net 1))
 (segment (start 107.8 70.8) (end 110.6 70.8) (width 0.2) (layer "F.Cu") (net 1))
 (segment (start 98.8 54.5) (end 98.55 54.25) (width 0.2) (layer "F.Cu") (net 1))
 (segment (start 98.525 69.75) (end 98.575 69.7) (width 0.2) (layer "F.Cu") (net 1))
 (segment (start 97.5 57.25) (end 98.525 57.25) (width 0.2) (layer "F.Cu") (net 1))
 (segment (start 98.8 58.475) (end 98.8 57.575) (width 0.2) (layer "F.Cu") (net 1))
 (segment (start 97.5 54.25) (end 98.525 54.25) (width 0.2) (layer "F.Cu") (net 1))
 (segment (start 99.075 67.8) (end 98.575 68.3) (width 0.2) (layer "F.Cu") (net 1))
 (segment (start 98.525 60.25) (end 98.8 59.975) (width 0.2) (layer "F.Cu") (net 1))
 (segment (start 98.8 59.975) (end 98.8 59.025) (width 0.2) (layer "F.Cu") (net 1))
 (segment (start 98.575 69.7) (end 98.575 68.3) (width 0.2) (layer "F.Cu") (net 1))
 (segment (start 97.5 69.75) (end 98.4 69.75) (width 0.2) (layer "F.Cu") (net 1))
 (segment (start 97.5 52.75) (end 98.525 52.75) (width 0.2) (layer "F.Cu") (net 1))
 (segment (start 112.843052 67) (end 111.243052 65.4) (width 0.2) (layer "F.Cu") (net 1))
 (segment (start 103.3 67.9) (end 103.2 67.8) (width 0.2) (layer "F.Cu") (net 1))
 (segment (start 97.5 61.75) (end 98.525 61.75) (width 0.2) (layer "F.Cu") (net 1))
 (segment (start 98.525 68.25) (end 98.575 68.2) (width 0.2) (layer "F.Cu") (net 1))
 (segment (start 112.1 69.3) (end 113.325 69.3) (width 0.2) (layer "F.Cu") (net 1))
 (segment (start 98.525 52.75) (end 98.8 52.475) (width 0.2) (layer "F.Cu") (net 1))
 (segment (start 111.5 62.35) (end 111.75 62.35) (width 0.2) (layer "F.Cu") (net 1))
 (segment (start 114.625 67) (end 112.843052 67) (width 0.2) (layer "F.Cu") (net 1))
 (segment (start 97.5 55.7) (end 97.5 55.75) (width 0.2) (layer "F.Cu") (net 1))
 (segment (start 111.75 62.35) (end 112.9 63.5) (width 0.2) (layer "F.Cu") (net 1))
 (segment (start 98.525 58.75) (end 98.8 58.475) (width 0.2) (layer "F.Cu") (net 1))
 (segment (start 98.8 52.475) (end 98.8 51.5) (width 0.2) (layer "F.Cu") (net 1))
 (segment (start 97.5 68.25) (end 98.525 68.25) (width 0.2) (layer "F.Cu") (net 1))
 (segment (start 97.5 60.25) (end 98.525 60.25) (width 0.2) (layer "F.Cu") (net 1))
 (segment (start 103.2 67.8) (end 99.075 67.8) (width 0.2) (layer "F.Cu") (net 1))
 (segment (start 98.8 57.575) (end 98.475 57.25) (width 0.2) (layer "F.Cu") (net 1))
 (segment (start 98.8 56.975) (end 98.8 56.025) (width 0.2) (layer "F.Cu") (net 1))
 (segment (start 108.2 50.7) (end 111.5 54) (width 0.2) (layer "F.Cu") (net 1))
 (segment (start 97.5 58.75) (end 98.525 58.75) (width 0.2) (layer "F.Cu") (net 1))
 (segment (start 98.8 56.025) (end 98.475 55.7) (width 0.2) (layer "F.Cu") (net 1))
 (segment (start 98.7 61.575) (end 98.7 60.6) (width 0.2) (layer "F.Cu") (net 1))
 (segment (start 111.5 54) (end 111.5 59) (width 0.2) (layer "F.Cu") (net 1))
 (segment (start 110.6 70.8) (end 112.1 69.3) (width 0.2) (layer "F.Cu") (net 1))
 (segment (start 98.8 55.475) (end 98.8 54.5) (width 0.2) (layer "F.Cu") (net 1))
 (segment (start 113.325 69.3) (end 114.625 70.6) (width 0.2) (layer "F.Cu") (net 1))
 (segment (start 98.475 57.25) (end 97.5 57.25) (width 0.2) (layer "F.Cu") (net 1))
 (via (at 103.3 67.9) (size 0.6) (drill 0.3) (layers "F.Cu" "B.Cu") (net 1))
 (via (at 112.9 63.5) (size 0.6) (drill 0.3) (layers "F.Cu" "B.Cu") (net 1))
 (segment (start 111.3 65.1) (end 111.3 65.4) (width 0.2) (layer "B.Cu") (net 1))
 (segment (start 103.3 67.9) (end 106.1 67.9) (width 0.2) (layer "B.Cu") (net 1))
 (segment (start 107.8 69.6) (end 107.8 70.8) (width 0.2) (layer "B.Cu") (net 1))
 (segment (start 112.9 63.5) (end 111.3 65.1) (width 0.2) (layer "B.Cu") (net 1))
 (segment (start 106.1 67.9) (end 107.8 69.6) (width 0.2) (layer "B.Cu") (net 1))
 (segment (start 109 64.5) (end 108.8 64.5) (width 0.2) (layer "F.Cu") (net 59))
 (segment (start 108.8 64.5) (end 107.555 65.745) (width 0.2) (layer "F.Cu") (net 59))
 (segment (start 107.555 66.6) (end 107.3 66.345) (width 0.2) (layer "F.Cu") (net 59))
 (segment (start 107.3 66.345) (end 107.3 60.25) (width 0.2) (layer "F.Cu") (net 59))
 (segment (start 107.555 65.745) (end 107.555 66.6) (width 0.2) (layer "F.Cu") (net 59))
 (segment (start 107.3 60.25) (end 108.55 59) (width 0.2) (layer "F.Cu") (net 59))
 (via (at 109 64.5) (size 0.6) (drill 0.3) (layers "F.Cu" "B.Cu") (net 59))
 (segment (start 109 64.5) (end 112.1 67.6) (width 0.2) (layer "B.Cu") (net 59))
 (segment (start 112.1 67.6) (end 112.1 68.2) (width 0.2) (layer "B.Cu") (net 59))
 (segment (start 107.8 67.5) (end 108.7 66.6) (width 0.2) (layer "F.Cu") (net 60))
 (segment (start 108.7 66.6) (end 110.5 64.8) (width 0.2) (layer "F.Cu") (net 60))
 (segment (start 113.5 64.1) (end 114.5 63.1) (width 0.2) (layer "F.Cu") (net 60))
 (segment (start 110.5 64.8) (end 111.2 64.1) (width 0.2) (layer "F.Cu") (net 60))
 (segment (start 107.8 68.8) (end 107.8 67.5) (width 0.2) (layer "F.Cu") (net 60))
 (segment (start 111.2 64.1) (end 113.5 64.1) (width 0.2) (layer "F.Cu") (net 60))
 (segment (start 110.5 64.8) (end 110.5 57.6) (width 0.2) (layer "F.Cu") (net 60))
 (segment (start 110.5 57.6) (end 108.2 55.3) (width 0.2) (layer "F.Cu") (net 60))
 (segment (start 112.2 65.4) (end 113.2 65.4) (width 0.2) (layer "F.Cu") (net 61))
 (segment (start 113.2 65.4) (end 113.3 65.3) (width 0.2) (layer "F.Cu") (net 61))
 (via (at 113.3 65.3) (size 0.6) (drill 0.3) (layers "F.Cu" "B.Cu") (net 61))
 (segment (start 114.4 64.2) (end 114.4 61.5) (width 0.2) (layer "B.Cu") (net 61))
 (segment (start 113.3 65.3) (end 114.4 64.2) (width 0.2) (layer "B.Cu") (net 61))
 (segment (start 106.075 69.5) (end 106.7 68.875) (width 0.2) (layer "F.Cu") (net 2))
 (segment (start 105.05 69.5) (end 106.075 69.5) (width 0.2) (layer "F.Cu") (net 2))
 (segment (start 106.7 68.875) (end 106.7 64.8) (width 0.2) (layer "F.Cu") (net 2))
 (via (at 106.7 64.8) (size 0.6) (drill 0.3) (layers "F.Cu" "B.Cu") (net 2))
 (segment (start 106.7 54.4) (end 108.1 53) (width 0.2) (layer "B.Cu") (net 2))
 (segment (start 108.5 63) (end 108.5 62.4) (width 0.2) (layer "B.Cu") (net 2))
 (segment (start 106.7 64.8) (end 108.5 63) (width 0.2) (layer "B.Cu") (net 2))
 (segment (start 106.7 64.8) (end 106.7 54.4) (width 0.2) (layer "B.Cu") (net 2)))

